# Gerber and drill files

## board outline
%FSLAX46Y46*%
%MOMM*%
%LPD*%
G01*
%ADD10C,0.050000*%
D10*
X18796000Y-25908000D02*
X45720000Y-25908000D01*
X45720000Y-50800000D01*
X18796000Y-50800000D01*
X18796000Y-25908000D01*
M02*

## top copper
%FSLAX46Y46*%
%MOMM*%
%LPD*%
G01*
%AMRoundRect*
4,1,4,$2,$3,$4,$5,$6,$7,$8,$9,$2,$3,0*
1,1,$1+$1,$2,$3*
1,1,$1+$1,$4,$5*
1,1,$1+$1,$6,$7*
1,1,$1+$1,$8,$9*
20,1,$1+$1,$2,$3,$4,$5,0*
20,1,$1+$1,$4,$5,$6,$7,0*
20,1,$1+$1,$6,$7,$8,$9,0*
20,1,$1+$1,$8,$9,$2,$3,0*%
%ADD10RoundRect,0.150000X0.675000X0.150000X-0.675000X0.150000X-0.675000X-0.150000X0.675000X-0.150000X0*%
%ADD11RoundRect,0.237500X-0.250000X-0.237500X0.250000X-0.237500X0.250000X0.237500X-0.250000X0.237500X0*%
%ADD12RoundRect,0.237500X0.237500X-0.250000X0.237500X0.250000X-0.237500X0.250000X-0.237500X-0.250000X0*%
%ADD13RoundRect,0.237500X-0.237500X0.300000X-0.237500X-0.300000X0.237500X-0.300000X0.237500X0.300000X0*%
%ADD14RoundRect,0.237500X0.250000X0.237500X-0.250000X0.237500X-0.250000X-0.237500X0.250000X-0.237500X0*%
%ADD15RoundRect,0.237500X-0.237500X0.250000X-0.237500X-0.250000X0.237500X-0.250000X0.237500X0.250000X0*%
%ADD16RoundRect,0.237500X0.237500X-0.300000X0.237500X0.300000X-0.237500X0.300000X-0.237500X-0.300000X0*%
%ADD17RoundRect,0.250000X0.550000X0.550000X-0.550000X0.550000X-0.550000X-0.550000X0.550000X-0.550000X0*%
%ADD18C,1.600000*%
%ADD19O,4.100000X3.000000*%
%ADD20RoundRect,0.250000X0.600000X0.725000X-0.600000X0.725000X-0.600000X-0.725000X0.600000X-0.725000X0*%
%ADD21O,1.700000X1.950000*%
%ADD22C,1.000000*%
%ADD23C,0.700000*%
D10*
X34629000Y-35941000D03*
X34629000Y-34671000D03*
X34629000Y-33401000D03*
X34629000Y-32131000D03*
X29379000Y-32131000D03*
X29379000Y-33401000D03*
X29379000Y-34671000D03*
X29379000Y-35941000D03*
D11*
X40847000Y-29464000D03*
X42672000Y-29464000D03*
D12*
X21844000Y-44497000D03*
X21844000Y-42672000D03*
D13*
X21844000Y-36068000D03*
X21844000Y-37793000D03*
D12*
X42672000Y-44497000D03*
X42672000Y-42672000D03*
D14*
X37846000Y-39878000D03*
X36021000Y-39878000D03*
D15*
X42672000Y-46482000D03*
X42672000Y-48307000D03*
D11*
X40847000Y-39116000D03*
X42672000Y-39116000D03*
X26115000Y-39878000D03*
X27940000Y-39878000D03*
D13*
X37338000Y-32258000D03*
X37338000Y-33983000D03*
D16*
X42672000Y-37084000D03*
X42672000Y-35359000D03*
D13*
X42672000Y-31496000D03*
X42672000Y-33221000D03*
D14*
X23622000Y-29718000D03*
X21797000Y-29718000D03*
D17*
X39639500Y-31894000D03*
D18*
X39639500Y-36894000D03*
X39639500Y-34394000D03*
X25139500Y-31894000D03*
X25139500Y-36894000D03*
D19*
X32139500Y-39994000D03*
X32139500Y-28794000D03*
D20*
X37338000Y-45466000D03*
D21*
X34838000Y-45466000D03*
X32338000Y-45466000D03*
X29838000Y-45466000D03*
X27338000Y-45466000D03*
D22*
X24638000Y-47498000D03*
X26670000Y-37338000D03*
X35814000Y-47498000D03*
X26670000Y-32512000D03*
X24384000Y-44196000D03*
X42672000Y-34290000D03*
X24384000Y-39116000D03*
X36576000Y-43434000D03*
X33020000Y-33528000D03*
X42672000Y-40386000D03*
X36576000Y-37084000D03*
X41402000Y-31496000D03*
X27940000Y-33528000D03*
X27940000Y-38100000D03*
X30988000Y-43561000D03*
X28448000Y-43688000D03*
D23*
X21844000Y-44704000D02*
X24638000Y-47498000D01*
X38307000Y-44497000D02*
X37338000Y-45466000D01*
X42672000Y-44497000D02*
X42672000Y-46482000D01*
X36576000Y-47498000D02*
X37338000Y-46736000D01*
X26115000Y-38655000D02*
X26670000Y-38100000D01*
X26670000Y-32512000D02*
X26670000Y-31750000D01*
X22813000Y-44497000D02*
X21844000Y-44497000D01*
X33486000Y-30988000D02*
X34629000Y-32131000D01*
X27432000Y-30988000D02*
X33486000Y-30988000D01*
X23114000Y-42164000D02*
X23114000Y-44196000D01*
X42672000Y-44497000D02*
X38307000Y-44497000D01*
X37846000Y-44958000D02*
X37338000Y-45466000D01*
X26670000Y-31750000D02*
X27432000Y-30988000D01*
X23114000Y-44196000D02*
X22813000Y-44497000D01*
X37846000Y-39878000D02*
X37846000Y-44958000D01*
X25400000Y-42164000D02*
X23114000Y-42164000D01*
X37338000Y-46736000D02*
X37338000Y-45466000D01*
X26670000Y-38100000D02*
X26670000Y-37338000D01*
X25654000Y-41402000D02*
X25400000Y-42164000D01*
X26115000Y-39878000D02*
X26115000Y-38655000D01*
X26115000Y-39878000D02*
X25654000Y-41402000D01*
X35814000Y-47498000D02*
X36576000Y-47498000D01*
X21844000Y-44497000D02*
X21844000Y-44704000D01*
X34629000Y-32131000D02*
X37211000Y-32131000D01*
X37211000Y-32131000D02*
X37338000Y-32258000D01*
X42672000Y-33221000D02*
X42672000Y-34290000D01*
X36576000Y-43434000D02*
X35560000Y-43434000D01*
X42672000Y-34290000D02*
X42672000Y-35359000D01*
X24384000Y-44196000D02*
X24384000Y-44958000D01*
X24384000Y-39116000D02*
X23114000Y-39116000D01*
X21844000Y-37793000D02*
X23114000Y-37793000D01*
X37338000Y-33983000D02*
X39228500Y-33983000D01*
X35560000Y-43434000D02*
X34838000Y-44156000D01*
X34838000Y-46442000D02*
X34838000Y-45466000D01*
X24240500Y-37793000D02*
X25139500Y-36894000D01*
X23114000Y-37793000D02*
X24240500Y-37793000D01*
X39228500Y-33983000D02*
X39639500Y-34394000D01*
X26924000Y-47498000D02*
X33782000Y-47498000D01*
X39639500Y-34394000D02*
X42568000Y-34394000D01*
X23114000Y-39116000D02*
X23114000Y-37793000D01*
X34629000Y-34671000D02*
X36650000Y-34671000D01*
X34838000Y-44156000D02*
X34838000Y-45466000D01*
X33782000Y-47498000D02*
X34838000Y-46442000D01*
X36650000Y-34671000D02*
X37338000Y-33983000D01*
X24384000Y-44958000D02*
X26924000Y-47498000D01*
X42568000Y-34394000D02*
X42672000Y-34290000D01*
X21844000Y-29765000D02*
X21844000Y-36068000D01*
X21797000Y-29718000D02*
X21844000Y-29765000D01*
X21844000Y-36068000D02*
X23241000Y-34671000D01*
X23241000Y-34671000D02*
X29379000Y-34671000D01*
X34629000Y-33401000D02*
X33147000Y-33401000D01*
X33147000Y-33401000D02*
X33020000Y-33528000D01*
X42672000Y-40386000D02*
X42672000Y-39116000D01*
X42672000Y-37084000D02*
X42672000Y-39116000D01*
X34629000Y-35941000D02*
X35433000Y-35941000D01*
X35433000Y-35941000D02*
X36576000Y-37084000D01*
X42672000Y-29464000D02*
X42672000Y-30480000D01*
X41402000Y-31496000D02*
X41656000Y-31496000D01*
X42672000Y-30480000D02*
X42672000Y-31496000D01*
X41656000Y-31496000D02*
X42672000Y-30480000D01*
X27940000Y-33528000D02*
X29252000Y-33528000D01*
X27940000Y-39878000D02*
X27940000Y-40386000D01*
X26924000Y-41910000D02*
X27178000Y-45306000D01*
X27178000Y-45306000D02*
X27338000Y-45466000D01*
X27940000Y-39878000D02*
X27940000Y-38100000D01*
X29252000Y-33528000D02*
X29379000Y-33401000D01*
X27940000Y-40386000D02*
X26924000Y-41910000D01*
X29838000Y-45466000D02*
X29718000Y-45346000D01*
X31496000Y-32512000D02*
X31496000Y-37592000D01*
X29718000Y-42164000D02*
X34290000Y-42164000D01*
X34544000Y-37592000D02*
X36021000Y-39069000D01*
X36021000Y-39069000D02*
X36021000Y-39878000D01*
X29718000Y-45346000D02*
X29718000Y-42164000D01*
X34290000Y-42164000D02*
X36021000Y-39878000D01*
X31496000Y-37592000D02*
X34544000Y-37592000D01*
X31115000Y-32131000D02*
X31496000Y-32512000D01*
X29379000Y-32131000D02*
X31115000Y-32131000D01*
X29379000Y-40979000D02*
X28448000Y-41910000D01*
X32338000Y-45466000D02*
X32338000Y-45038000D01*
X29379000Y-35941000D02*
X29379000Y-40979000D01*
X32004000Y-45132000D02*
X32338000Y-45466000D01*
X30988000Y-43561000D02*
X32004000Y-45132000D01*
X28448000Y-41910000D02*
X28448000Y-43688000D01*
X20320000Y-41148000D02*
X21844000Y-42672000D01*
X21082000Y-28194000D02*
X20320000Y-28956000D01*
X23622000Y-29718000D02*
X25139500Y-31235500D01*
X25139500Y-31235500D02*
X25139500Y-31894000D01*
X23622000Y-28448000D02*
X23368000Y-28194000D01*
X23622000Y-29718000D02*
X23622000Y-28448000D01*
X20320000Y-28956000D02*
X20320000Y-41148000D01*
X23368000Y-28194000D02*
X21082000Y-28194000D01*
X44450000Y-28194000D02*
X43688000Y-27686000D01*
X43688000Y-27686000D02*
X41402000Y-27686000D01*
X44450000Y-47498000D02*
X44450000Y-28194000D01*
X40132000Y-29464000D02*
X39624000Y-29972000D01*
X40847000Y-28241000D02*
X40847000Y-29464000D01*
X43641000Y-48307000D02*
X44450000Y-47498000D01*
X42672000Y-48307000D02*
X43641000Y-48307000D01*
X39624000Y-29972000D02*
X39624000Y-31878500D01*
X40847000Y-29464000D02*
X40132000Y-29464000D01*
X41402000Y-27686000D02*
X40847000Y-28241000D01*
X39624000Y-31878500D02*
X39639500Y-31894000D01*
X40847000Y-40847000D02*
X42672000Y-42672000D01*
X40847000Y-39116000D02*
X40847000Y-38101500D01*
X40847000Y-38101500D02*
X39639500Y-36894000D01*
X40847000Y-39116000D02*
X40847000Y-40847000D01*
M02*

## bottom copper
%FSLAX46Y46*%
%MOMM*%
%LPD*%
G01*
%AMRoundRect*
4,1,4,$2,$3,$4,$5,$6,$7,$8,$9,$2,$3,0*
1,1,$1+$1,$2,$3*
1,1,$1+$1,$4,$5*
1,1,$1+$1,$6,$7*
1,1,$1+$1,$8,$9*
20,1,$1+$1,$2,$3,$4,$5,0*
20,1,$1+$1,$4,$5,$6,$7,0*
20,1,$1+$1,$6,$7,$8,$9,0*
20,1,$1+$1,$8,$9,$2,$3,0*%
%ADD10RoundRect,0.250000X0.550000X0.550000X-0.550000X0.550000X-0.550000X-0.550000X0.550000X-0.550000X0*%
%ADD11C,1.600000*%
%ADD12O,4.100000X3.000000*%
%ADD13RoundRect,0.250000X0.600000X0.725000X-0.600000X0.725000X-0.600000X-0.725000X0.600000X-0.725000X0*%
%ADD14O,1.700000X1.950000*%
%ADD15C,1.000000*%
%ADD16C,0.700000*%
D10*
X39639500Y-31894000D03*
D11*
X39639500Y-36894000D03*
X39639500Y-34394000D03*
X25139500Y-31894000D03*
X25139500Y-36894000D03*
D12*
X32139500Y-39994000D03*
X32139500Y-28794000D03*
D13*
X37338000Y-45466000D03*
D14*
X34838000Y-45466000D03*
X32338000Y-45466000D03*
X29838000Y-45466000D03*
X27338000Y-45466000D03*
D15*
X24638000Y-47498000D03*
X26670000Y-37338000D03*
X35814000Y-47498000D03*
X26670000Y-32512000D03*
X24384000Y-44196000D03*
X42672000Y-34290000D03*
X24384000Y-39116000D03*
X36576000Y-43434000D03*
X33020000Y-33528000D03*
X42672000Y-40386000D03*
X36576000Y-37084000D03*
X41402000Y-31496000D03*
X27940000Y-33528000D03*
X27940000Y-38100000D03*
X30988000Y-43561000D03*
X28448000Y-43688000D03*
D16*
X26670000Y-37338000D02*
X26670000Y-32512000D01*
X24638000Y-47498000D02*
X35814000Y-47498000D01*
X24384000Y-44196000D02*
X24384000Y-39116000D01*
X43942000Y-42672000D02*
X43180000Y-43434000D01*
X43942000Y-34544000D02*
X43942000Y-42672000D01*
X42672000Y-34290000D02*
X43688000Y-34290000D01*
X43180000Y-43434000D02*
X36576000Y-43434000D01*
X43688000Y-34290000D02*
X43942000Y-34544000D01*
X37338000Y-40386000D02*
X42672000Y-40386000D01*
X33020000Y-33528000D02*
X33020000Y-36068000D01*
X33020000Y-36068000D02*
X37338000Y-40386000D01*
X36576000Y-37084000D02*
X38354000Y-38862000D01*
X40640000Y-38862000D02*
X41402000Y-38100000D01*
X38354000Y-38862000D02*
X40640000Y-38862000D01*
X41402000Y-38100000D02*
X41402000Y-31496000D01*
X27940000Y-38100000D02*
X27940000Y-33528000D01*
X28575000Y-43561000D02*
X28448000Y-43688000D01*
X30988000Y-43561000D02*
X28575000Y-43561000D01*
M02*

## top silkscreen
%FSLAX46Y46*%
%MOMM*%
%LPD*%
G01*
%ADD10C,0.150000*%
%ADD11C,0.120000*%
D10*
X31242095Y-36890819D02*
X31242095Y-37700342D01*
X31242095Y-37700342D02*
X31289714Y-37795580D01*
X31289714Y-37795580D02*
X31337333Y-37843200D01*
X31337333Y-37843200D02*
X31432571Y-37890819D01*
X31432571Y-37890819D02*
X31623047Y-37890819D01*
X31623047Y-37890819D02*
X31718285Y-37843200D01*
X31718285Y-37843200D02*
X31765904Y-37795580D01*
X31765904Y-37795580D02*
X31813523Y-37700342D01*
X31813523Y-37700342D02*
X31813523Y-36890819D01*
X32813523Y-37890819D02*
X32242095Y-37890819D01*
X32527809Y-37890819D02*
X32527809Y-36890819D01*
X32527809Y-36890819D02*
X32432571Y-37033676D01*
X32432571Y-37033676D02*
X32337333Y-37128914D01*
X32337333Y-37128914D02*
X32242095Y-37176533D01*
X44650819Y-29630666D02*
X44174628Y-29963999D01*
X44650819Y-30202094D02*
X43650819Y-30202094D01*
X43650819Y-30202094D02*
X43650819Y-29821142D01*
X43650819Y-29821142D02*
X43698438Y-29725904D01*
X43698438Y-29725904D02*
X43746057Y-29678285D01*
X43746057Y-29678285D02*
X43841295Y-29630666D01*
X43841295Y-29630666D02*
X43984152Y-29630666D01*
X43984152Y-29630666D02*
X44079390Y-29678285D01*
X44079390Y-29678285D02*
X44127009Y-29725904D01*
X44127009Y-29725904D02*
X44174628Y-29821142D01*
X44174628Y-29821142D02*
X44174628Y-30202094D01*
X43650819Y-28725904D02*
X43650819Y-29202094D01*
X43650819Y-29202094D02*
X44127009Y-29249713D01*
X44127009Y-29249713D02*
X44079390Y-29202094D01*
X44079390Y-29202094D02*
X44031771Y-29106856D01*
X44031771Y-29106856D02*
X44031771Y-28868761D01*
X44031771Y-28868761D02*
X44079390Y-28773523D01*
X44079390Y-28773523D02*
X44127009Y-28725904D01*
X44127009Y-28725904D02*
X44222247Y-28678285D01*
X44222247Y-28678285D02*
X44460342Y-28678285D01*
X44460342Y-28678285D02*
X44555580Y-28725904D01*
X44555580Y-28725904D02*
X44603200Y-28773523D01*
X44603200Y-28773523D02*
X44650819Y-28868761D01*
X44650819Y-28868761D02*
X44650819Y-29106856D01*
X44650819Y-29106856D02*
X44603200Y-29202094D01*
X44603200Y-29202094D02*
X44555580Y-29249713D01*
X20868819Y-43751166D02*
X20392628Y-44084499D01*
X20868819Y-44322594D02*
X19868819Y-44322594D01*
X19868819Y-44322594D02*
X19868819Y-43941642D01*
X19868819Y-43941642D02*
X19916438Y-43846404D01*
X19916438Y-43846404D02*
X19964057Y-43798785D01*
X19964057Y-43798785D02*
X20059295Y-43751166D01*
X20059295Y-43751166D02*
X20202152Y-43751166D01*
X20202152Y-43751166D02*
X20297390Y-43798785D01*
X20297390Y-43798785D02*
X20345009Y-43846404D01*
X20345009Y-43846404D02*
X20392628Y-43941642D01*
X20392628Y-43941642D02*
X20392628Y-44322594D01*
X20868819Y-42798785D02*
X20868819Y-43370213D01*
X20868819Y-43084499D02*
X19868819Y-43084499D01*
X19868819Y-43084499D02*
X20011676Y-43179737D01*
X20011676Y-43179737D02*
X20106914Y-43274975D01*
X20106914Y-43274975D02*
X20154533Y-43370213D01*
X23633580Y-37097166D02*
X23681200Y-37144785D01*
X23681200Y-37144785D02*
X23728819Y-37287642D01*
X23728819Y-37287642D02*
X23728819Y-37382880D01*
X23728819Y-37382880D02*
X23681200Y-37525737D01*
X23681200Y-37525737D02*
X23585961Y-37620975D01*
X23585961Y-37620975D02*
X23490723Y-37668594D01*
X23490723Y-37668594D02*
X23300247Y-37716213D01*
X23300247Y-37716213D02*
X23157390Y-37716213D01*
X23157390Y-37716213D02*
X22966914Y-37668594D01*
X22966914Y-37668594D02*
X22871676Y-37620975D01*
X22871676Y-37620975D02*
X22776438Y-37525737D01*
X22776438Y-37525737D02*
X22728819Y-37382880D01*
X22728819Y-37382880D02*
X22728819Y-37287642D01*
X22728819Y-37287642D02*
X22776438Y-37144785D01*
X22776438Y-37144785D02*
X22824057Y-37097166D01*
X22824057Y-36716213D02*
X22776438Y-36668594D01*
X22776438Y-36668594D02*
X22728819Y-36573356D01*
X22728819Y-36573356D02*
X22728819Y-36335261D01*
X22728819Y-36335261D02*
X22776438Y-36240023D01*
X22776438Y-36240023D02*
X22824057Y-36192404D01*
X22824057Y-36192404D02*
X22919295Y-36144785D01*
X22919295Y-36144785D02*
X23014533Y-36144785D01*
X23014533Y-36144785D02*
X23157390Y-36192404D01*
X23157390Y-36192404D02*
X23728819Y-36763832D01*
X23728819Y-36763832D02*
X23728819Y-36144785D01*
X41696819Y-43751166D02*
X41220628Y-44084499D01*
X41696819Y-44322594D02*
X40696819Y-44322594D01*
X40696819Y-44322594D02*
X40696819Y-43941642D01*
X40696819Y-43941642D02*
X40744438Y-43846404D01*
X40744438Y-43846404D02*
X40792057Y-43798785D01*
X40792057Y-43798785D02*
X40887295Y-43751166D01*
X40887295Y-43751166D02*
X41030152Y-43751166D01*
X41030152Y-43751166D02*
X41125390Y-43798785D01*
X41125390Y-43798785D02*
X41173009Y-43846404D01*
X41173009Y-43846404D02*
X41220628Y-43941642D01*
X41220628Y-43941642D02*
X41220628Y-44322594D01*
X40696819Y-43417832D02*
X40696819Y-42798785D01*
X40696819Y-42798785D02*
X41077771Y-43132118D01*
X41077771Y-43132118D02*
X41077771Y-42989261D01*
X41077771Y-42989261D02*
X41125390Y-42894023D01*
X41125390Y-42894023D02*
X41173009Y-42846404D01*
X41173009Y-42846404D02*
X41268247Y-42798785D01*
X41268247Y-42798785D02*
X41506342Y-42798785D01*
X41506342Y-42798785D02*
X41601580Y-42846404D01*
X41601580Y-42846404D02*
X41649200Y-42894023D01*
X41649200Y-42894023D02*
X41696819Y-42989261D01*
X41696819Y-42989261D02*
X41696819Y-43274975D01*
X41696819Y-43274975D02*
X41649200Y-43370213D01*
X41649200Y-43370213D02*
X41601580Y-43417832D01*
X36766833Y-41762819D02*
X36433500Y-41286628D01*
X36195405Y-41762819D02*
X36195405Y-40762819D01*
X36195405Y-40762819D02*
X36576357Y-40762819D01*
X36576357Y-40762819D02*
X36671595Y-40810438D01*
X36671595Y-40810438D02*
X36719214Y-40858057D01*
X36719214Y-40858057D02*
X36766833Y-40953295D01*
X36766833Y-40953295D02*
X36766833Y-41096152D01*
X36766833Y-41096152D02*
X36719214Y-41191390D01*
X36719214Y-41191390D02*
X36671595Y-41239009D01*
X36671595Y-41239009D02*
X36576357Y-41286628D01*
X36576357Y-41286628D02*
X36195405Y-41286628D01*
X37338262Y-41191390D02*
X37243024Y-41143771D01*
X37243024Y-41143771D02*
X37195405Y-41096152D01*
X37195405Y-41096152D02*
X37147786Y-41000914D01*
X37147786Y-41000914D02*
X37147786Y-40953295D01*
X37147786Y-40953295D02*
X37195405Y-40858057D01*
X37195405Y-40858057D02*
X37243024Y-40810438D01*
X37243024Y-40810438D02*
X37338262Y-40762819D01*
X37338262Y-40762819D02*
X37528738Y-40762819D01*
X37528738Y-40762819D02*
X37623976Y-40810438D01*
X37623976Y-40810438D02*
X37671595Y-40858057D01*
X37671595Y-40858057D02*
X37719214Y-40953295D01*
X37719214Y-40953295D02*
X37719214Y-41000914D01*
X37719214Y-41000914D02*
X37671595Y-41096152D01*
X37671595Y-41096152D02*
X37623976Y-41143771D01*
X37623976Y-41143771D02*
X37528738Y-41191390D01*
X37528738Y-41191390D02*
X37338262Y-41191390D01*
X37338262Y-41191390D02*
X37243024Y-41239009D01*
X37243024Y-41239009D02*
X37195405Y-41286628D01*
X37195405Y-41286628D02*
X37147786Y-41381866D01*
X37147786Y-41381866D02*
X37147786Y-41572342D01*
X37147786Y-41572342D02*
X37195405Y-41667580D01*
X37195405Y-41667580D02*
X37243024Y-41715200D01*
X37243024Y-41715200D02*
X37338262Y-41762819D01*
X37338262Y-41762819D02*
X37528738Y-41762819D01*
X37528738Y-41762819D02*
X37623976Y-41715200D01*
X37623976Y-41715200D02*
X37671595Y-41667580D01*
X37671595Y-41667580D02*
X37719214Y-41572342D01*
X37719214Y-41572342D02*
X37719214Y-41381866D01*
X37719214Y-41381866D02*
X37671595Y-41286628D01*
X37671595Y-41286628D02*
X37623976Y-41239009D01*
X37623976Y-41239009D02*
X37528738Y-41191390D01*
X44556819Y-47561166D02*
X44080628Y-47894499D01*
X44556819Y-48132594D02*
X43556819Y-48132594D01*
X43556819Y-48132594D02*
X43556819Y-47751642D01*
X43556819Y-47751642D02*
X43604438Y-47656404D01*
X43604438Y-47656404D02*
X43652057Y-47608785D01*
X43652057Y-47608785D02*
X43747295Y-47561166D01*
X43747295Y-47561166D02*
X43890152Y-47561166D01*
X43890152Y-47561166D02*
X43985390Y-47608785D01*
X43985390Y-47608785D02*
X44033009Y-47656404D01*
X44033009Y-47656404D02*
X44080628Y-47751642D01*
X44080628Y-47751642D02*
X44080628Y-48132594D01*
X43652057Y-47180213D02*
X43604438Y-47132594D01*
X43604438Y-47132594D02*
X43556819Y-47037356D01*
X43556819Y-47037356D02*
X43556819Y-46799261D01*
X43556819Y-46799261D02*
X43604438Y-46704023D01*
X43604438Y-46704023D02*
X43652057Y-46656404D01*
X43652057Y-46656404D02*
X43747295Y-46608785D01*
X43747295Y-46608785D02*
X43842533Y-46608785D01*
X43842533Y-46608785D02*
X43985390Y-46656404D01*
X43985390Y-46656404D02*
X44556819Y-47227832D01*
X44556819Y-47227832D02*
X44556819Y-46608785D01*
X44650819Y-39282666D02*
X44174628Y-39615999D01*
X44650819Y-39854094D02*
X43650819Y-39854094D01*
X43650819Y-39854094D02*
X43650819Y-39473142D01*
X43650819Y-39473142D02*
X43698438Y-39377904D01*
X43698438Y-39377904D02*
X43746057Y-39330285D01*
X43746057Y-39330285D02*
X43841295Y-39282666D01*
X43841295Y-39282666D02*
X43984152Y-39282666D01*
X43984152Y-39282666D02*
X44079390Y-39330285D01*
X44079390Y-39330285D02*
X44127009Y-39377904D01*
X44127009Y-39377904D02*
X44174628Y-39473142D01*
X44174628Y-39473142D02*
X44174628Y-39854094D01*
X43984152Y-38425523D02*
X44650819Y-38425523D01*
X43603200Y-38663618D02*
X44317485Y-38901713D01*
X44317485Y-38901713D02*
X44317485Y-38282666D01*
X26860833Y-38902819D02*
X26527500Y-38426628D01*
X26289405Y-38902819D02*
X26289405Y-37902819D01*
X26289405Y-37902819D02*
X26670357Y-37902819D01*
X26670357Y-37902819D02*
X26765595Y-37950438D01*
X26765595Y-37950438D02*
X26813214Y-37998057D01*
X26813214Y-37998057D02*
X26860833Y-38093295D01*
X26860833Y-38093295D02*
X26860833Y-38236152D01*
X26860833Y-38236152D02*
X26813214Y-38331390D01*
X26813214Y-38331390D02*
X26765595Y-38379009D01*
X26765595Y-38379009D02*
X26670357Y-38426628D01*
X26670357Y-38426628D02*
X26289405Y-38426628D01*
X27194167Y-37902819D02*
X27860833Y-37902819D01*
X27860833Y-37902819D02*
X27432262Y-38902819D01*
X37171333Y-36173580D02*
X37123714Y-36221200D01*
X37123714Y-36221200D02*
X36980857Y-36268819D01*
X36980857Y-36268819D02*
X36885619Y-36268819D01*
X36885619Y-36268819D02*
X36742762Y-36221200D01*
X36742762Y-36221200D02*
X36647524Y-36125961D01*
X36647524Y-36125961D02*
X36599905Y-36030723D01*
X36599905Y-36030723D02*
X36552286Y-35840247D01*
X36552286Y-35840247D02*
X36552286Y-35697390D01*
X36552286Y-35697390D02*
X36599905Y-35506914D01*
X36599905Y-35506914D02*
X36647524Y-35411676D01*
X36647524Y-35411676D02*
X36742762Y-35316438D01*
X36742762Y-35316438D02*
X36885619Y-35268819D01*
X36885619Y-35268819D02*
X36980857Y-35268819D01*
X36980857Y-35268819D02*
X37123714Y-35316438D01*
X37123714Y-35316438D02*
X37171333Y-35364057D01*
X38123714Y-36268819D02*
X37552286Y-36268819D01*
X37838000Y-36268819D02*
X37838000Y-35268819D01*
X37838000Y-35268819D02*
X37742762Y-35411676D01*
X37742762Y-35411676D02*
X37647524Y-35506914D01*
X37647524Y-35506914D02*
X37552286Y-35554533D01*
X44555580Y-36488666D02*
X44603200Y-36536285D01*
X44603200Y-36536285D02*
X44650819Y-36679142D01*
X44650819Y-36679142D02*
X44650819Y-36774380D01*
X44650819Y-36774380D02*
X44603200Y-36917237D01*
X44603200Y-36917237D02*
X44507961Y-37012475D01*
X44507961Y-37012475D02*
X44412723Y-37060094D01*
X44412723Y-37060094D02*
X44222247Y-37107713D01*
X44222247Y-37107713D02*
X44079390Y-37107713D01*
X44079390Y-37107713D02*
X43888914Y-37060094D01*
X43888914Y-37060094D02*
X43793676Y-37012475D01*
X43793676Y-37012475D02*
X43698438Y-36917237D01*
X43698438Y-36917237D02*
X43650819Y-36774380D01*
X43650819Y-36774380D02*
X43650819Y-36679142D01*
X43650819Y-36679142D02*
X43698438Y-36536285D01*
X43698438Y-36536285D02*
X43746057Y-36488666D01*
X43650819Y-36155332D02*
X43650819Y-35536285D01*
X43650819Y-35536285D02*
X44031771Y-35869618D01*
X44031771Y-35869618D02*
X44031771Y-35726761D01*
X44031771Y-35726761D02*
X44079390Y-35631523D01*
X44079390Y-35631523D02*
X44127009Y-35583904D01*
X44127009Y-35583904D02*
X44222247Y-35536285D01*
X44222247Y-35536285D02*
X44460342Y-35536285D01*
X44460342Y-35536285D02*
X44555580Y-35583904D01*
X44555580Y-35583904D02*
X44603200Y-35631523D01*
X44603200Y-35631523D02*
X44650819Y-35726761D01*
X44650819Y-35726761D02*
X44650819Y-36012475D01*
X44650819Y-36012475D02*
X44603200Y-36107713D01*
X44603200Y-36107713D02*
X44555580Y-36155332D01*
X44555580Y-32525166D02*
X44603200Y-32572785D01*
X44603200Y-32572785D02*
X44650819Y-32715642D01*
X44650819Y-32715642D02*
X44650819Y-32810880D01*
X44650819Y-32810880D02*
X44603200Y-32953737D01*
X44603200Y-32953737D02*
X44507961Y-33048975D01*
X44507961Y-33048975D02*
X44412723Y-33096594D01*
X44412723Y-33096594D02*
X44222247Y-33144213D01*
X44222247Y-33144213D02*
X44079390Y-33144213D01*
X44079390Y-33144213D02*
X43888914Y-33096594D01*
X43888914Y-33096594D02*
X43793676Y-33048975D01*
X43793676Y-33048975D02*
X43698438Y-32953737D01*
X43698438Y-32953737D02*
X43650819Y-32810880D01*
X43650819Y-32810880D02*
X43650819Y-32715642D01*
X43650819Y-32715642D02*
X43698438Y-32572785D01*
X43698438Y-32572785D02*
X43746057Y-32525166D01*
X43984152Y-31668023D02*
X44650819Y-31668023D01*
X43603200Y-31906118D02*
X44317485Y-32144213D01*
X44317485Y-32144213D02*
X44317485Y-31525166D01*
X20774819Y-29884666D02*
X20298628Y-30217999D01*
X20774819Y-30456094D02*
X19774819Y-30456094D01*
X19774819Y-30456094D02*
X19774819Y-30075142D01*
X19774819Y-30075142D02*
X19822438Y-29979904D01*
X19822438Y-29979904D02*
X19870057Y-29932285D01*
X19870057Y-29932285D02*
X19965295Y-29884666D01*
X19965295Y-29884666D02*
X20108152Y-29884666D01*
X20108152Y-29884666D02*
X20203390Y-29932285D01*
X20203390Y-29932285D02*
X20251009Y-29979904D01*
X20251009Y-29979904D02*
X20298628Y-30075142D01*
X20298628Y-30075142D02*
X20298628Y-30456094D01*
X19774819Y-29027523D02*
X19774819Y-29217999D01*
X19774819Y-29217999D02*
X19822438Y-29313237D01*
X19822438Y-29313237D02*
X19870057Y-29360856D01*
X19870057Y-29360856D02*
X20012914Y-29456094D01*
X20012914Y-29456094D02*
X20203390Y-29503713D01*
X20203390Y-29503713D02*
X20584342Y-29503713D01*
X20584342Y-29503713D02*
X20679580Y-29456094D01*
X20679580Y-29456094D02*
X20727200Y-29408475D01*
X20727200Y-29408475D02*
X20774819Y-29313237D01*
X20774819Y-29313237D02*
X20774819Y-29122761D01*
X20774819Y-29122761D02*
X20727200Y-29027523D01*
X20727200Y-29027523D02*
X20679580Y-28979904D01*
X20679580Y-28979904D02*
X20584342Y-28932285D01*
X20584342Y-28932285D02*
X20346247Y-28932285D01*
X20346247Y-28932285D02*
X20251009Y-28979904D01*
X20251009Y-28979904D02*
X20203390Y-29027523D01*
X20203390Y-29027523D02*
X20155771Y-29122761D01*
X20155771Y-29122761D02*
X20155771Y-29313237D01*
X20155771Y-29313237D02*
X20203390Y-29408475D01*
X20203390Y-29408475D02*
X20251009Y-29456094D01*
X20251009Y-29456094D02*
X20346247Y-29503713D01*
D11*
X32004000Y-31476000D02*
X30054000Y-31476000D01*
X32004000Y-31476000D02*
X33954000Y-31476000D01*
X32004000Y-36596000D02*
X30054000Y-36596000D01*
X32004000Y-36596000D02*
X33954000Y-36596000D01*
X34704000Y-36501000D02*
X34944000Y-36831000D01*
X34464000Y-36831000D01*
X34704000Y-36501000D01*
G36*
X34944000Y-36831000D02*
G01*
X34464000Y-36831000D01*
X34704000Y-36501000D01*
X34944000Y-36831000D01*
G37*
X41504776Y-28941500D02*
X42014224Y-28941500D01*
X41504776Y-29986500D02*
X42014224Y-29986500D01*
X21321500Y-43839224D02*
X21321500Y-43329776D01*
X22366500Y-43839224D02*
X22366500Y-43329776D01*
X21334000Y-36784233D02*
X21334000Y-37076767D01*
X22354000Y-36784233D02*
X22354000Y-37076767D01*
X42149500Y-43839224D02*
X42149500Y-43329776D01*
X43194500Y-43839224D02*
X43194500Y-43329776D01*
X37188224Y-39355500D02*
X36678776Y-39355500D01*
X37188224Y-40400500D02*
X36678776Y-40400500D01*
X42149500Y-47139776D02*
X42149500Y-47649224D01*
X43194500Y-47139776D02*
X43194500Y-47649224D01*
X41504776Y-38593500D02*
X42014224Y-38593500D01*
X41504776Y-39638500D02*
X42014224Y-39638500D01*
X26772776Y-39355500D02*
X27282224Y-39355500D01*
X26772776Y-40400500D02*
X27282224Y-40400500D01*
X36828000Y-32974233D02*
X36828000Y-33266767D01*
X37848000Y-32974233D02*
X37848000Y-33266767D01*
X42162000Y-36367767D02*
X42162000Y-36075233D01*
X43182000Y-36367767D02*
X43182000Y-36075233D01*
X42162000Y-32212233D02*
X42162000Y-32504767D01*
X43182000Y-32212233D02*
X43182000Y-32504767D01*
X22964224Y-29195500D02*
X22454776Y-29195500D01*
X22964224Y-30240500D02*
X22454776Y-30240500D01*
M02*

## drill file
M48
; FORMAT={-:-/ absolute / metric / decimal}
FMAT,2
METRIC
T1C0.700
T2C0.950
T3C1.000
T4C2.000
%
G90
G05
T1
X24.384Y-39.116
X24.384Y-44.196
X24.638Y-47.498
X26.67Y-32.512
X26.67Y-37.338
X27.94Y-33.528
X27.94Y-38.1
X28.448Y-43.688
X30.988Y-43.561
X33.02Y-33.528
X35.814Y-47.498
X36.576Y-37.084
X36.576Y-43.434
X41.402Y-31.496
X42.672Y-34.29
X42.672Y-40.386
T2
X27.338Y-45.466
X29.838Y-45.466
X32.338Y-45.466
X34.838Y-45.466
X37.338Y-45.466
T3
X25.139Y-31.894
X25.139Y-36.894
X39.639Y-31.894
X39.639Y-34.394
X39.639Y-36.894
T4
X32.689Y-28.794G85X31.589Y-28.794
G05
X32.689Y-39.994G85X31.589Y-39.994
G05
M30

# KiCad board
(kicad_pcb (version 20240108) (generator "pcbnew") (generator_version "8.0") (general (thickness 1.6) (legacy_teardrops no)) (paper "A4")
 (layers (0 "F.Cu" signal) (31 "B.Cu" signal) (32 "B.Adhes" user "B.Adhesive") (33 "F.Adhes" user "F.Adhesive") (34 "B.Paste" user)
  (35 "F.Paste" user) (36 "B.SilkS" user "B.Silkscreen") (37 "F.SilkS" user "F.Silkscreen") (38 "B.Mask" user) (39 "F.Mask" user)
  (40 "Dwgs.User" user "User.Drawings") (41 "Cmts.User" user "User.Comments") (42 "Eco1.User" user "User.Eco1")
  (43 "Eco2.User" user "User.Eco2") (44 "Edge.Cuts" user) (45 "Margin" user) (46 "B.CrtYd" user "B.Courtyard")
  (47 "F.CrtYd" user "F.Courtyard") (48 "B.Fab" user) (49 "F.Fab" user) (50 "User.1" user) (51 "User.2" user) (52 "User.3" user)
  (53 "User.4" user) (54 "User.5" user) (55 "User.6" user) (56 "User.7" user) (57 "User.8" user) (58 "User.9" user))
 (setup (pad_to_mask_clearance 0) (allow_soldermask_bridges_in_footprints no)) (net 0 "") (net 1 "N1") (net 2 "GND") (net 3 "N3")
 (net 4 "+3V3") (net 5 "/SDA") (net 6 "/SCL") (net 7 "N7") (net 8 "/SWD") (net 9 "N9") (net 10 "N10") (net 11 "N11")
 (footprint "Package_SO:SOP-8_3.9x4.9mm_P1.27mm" (layer "F.Cu") (at 32.004 34.036 180)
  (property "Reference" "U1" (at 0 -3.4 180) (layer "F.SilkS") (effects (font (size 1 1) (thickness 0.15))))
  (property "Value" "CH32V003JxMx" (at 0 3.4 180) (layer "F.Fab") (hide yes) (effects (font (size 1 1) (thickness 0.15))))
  (fp_line (start 0 2.56) (end 1.95 2.56) (stroke (width 0.12) (type solid)) (layer "F.SilkS"))
  (fp_line (start 0 2.56) (end -1.95 2.56) (stroke (width 0.12) (type solid)) (layer "F.SilkS"))
  (fp_line (start 0 -2.56) (end 1.95 -2.56) (stroke (width 0.12) (type solid)) (layer "F.SilkS"))
  (fp_line (start 0 -2.56) (end -1.95 -2.56) (stroke (width 0.12) (type solid)) (layer "F.SilkS"))
  (fp_poly
   (pts (xy -2.7 -2.465) (xy -2.94 -2.795) (xy -2.46 -2.795) (xy -2.7 -2.465)) (stroke (width 0.12) (type solid)) (fill solid)
   (layer "F.SilkS"))
  (pad "1" smd roundrect (at -2.625 -1.905 180) (size 1.65 0.6) (layers "F.Cu" "F.Paste" "F.Mask") (roundrect_rratio 0.25) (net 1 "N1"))
  (pad "2" smd roundrect (at -2.625 -0.635 180) (size 1.65 0.6) (layers "F.Cu" "F.Paste" "F.Mask") (roundrect_rratio 0.25) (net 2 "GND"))
  (pad "3" smd roundrect (at -2.625 0.635 180) (size 1.65 0.6) (layers "F.Cu" "F.Paste" "F.Mask") (roundrect_rratio 0.25) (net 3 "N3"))
  (pad "4" smd roundrect (at -2.625 1.905 180) (size 1.65 0.6) (layers "F.Cu" "F.Paste" "F.Mask") (roundrect_rratio 0.25) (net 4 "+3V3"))
  (pad "5" smd roundrect (at 2.625 1.905 180) (size 1.65 0.6) (layers "F.Cu" "F.Paste" "F.Mask") (roundrect_rratio 0.25) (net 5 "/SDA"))
  (pad "6" smd roundrect (at 2.625 0.635 180) (size 1.65 0.6) (layers "F.Cu" "F.Paste" "F.Mask") (roundrect_rratio 0.25) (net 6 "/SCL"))
  (pad "7" smd roundrect (at 2.625 -0.635 180) (size 1.65 0.6) (layers "F.Cu" "F.Paste" "F.Mask") (roundrect_rratio 0.25) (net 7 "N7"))
  (pad "8" smd roundrect (at 2.625 -1.905 180) (size 1.65 0.6) (layers "F.Cu" "F.Paste" "F.Mask") (roundrect_rratio 0.25) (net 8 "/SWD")))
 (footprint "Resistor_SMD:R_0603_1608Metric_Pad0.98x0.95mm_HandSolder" (layer "F.Cu") (at 41.7595 29.464)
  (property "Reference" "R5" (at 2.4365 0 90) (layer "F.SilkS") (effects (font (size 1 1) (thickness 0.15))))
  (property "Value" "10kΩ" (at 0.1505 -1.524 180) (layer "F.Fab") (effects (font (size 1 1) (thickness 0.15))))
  (fp_line (start -0.254724 -0.5225) (end 0.254724 -0.5225) (stroke (width 0.12) (type solid)) (layer "F.SilkS"))
  (fp_line (start -0.254724 0.5225) (end 0.254724 0.5225) (stroke (width 0.12) (type solid)) (layer "F.SilkS"))
  (pad "1" smd roundrect (at -0.9125 0) (size 0.975 0.95) (layers "F.Cu" "F.Paste" "F.Mask") (roundrect_rratio 0.25) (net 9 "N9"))
  (pad "2" smd roundrect (at 0.9125 0) (size 0.975 0.95) (layers "F.Cu" "F.Paste" "F.Mask") (roundrect_rratio 0.25) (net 1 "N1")))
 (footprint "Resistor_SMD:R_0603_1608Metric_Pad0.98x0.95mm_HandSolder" (layer "F.Cu") (at 21.844 43.5845 90)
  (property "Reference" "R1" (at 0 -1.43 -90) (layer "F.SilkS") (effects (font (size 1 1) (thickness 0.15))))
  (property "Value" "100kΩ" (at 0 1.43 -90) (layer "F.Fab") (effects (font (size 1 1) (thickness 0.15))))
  (fp_line (start -0.254724 -0.5225) (end 0.254724 -0.5225) (stroke (width 0.12) (type solid)) (layer "F.SilkS"))
  (fp_line (start -0.254724 0.5225) (end 0.254724 0.5225) (stroke (width 0.12) (type solid)) (layer "F.SilkS"))
  (pad "1" smd roundrect (at -0.9125 0 90) (size 0.975 0.95) (layers "F.Cu" "F.Paste" "F.Mask") (roundrect_rratio 0.25) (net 4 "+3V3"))
  (pad "2" smd roundrect (at 0.9125 0 90) (size 0.975 0.95) (layers "F.Cu" "F.Paste" "F.Mask") (roundrect_rratio 0.25) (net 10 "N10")))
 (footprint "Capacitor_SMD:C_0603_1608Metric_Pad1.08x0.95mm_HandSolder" (layer "F.Cu") (at 21.844 36.9305 -90)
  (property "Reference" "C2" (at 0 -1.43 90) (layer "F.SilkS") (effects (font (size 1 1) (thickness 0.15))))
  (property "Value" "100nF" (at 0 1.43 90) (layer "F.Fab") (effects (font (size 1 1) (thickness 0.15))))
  (fp_line (start -0.146267 0.51) (end 0.146267 0.51) (stroke (width 0.12) (type solid)) (layer "F.SilkS"))
  (fp_line (start -0.146267 -0.51) (end 0.146267 -0.51) (stroke (width 0.12) (type solid)) (layer "F.SilkS"))
  (pad "1" smd roundrect (at -0.8625 0 270) (size 1.075 0.95) (layers "F.Cu" "F.Paste" "F.Mask") (roundrect_rratio 0.25) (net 7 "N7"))
  (pad "2" smd roundrect (at 0.8625 0 270) (size 1.075 0.95) (layers "F.Cu" "F.Paste" "F.Mask") (roundrect_rratio 0.25) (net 2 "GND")))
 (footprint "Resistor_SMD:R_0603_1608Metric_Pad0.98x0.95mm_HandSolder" (layer "F.Cu") (at 42.672 43.5845 90)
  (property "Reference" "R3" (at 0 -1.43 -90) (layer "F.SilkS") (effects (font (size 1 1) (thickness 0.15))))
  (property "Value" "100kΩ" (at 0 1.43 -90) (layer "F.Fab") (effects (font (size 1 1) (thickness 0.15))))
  (fp_line (start -0.254724 -0.5225) (end 0.254724 -0.5225) (stroke (width 0.12) (type solid)) (layer "F.SilkS"))
  (fp_line (start -0.254724 0.5225) (end 0.254724 0.5225) (stroke (width 0.12) (type solid)) (layer "F.SilkS"))
  (pad "1" smd roundrect (at -0.9125 0 90) (size 0.975 0.95) (layers "F.Cu" "F.Paste" "F.Mask") (roundrect_rratio 0.25) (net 4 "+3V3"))
  (pad "2" smd roundrect (at 0.9125 0 90) (size 0.975 0.95) (layers "F.Cu" "F.Paste" "F.Mask") (roundrect_rratio 0.25) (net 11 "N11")))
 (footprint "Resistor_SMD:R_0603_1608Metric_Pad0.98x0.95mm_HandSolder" (layer "F.Cu") (at 36.9335 39.878 180)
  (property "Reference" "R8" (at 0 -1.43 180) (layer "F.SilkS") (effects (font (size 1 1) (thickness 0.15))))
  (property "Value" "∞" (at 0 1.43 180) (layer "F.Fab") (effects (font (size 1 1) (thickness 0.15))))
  (fp_line (start -0.254724 0.5225) (end 0.254724 0.5225) (stroke (width 0.12) (type solid)) (layer "F.SilkS"))
  (fp_line (start -0.254724 -0.5225) (end 0.254724 -0.5225) (stroke (width 0.12) (type solid)) (layer "F.SilkS"))
  (pad "1" smd roundrect (at -0.9125 0 180) (size 0.975 0.95) (layers "F.Cu" "F.Paste" "F.Mask") (roundrect_rratio 0.25) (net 4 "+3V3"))
  (pad "2" smd roundrect (at 0.9125 0 180) (size 0.975 0.95) (layers "F.Cu" "F.Paste" "F.Mask") (roundrect_rratio 0.25) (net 5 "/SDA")))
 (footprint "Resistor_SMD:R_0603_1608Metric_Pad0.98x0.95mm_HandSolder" (layer "F.Cu") (at 42.672 47.3945 -90)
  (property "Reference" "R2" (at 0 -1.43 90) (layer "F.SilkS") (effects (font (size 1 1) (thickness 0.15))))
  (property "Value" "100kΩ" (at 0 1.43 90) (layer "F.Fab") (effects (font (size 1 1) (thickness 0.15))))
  (fp_line (start -0.254724 0.5225) (end 0.254724 0.5225) (stroke (width 0.12) (type solid)) (layer "F.SilkS"))
  (fp_line (start -0.254724 -0.5225) (end 0.254724 -0.5225) (stroke (width 0.12) (type solid)) (layer "F.SilkS"))
  (pad "1" smd roundrect (at -0.9125 0 270) (size 0.975 0.95) (layers "F.Cu" "F.Paste" "F.Mask") (roundrect_rratio 0.25) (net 4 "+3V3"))
  (pad "2" smd roundrect (at 0.9125 0 270) (size 0.975 0.95) (layers "F.Cu" "F.Paste" "F.Mask") (roundrect_rratio 0.25) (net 9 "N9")))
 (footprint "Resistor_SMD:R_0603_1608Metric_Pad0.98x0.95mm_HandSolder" (layer "F.Cu") (at 41.7595 39.116)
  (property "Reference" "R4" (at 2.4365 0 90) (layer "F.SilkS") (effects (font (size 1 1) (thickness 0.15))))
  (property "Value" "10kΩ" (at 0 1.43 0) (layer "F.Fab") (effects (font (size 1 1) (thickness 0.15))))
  (fp_line (start -0.254724 -0.5225) (end 0.254724 -0.5225) (stroke (width 0.12) (type solid)) (layer "F.SilkS"))
  (fp_line (start -0.254724 0.5225) (end 0.254724 0.5225) (stroke (width 0.12) (type solid)) (layer "F.SilkS"))
  (pad "1" smd roundrect (at -0.9125 0) (size 0.975 0.95) (layers "F.Cu" "F.Paste" "F.Mask") (roundrect_rratio 0.25) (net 11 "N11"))
  (pad "2" smd roundrect (at 0.9125 0) (size 0.975 0.95) (layers "F.Cu" "F.Paste" "F.Mask") (roundrect_rratio 0.25) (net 3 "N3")))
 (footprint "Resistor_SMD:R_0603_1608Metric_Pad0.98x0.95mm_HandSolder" (layer "F.Cu") (at 27.0275 39.878)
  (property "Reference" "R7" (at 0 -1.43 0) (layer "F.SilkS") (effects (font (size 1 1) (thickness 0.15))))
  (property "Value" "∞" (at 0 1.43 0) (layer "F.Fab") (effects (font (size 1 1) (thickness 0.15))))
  (fp_line (start -0.254724 -0.5225) (end 0.254724 -0.5225) (stroke (width 0.12) (type solid)) (layer "F.SilkS"))
  (fp_line (start -0.254724 0.5225) (end 0.254724 0.5225) (stroke (width 0.12) (type solid)) (layer "F.SilkS"))
  (pad "1" smd roundrect (at -0.9125 0) (size 0.975 0.95) (layers "F.Cu" "F.Paste" "F.Mask") (roundrect_rratio 0.25) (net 4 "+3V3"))
  (pad "2" smd roundrect (at 0.9125 0) (size 0.975 0.95) (layers "F.Cu" "F.Paste" "F.Mask") (roundrect_rratio 0.25) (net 6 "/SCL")))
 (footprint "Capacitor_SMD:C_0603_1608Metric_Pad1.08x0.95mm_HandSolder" (layer "F.Cu") (at 37.338 33.1205 -90)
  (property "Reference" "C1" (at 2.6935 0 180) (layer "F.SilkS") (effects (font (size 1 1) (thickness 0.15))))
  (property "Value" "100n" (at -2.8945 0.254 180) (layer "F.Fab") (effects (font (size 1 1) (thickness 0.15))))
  (fp_line (start -0.146267 0.51) (end 0.146267 0.51) (stroke (width 0.12) (type solid)) (layer "F.SilkS"))
  (fp_line (start -0.146267 -0.51) (end 0.146267 -0.51) (stroke (width 0.12) (type solid)) (layer "F.SilkS"))
  (pad "1" smd roundrect (at -0.8625 0 270) (size 1.075 0.95) (layers "F.Cu" "F.Paste" "F.Mask") (roundrect_rratio 0.25) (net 4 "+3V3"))
  (pad "2" smd roundrect (at 0.8625 0 270) (size 1.075 0.95) (layers "F.Cu" "F.Paste" "F.Mask") (roundrect_rratio 0.25) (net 2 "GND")))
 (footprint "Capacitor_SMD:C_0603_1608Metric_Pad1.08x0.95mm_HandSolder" (layer "F.Cu") (at 42.672 36.2215 90)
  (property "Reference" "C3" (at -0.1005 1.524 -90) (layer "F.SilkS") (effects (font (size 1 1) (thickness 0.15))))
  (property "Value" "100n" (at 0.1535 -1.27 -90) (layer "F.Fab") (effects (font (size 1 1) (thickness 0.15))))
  (fp_line (start -0.146267 -0.51) (end 0.146267 -0.51) (stroke (width 0.12) (type solid)) (layer "F.SilkS"))
  (fp_line (start -0.146267 0.51) (end 0.146267 0.51) (stroke (width 0.12) (type solid)) (layer "F.SilkS"))
  (pad "1" smd roundrect (at -0.8625 0 90) (size 1.075 0.95) (layers "F.Cu" "F.Paste" "F.Mask") (roundrect_rratio 0.25) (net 3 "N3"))
  (pad "2" smd roundrect (at 0.8625 0 90) (size 1.075 0.95) (layers "F.Cu" "F.Paste" "F.Mask") (roundrect_rratio 0.25) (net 2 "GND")))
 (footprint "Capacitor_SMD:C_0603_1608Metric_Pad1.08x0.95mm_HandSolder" (layer "F.Cu") (at 42.672 32.3585 -90)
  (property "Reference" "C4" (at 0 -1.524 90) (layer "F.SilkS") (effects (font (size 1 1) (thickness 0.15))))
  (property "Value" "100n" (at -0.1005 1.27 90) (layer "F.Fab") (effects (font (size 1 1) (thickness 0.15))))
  (fp_line (start -0.146267 0.51) (end 0.146267 0.51) (stroke (width 0.12) (type solid)) (layer "F.SilkS"))
  (fp_line (start -0.146267 -0.51) (end 0.146267 -0.51) (stroke (width 0.12) (type solid)) (layer "F.SilkS"))
  (pad "1" smd roundrect (at -0.8625 0 270) (size 1.075 0.95) (layers "F.Cu" "F.Paste" "F.Mask") (roundrect_rratio 0.25) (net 1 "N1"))
  (pad "2" smd roundrect (at 0.8625 0 270) (size 1.075 0.95) (layers "F.Cu" "F.Paste" "F.Mask") (roundrect_rratio 0.25) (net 2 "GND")))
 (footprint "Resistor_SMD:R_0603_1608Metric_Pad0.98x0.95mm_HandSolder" (layer "F.Cu") (at 22.7095 29.718 180)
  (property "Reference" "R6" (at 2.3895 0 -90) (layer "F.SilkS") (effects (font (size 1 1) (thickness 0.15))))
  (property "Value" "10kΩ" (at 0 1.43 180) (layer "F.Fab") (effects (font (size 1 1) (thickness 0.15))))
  (fp_line (start -0.254724 0.5225) (end 0.254724 0.5225) (stroke (width 0.12) (type solid)) (layer "F.SilkS"))
  (fp_line (start -0.254724 -0.5225) (end 0.254724 -0.5225) (stroke (width 0.12) (type solid)) (layer "F.SilkS"))
  (pad "1" smd roundrect (at -0.9125 0 180) (size 0.975 0.95) (layers "F.Cu" "F.Paste" "F.Mask") (roundrect_rratio 0.25) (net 10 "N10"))
  (pad "2" smd roundrect (at 0.9125 0 180) (size 0.975 0.95) (layers "F.Cu" "F.Paste" "F.Mask") (roundrect_rratio 0.25) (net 7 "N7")))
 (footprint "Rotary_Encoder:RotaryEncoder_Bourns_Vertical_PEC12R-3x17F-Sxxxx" (layer "B.Cu") (at 39.6395 31.894 180)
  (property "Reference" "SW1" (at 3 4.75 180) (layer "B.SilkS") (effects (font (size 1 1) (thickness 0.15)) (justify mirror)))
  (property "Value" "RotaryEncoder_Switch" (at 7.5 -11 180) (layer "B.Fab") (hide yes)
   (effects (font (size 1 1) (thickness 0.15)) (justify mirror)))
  (pad "A" thru_hole roundrect (at 0 0 180) (size 1.6 1.6) (drill 1) (layers "*.Cu" "*.Mask") (remove_unused_layers no)
   (roundrect_rratio 0.15625) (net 9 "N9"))
  (pad "B" thru_hole circle (at 0 -5 180) (size 1.6 1.6) (drill 1) (layers "*.Cu" "*.Mask") (remove_unused_layers no) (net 11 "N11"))
  (pad "C" thru_hole circle (at 0 -2.5 180) (size 1.6 1.6) (drill 1) (layers "*.Cu" "*.Mask") (remove_unused_layers no) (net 2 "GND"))
  (pad "S1" thru_hole circle (at 14.5 0 180) (size 1.6 1.6) (drill 1) (layers "*.Cu" "*.Mask") (remove_unused_layers no) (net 10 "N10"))
  (pad "S2" thru_hole circle (at 14.5 -5 180) (size 1.6 1.6) (drill 1) (layers "*.Cu" "*.Mask") (remove_unused_layers no) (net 2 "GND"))
  (pad "SH" thru_hole oval (at 7.5 -8.1 180) (size 4.1 3) (drill oval 3.1 2) (layers "*.Cu" "*.Mask") (remove_unused_layers no))
  (pad "SH" thru_hole oval (at 7.5 3.1 180) (size 4.1 3) (drill oval 3.1 2) (layers "*.Cu" "*.Mask") (remove_unused_layers no)))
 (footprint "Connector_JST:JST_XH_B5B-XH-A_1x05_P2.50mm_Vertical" (layer "B.Cu") (at 37.338 45.466 180)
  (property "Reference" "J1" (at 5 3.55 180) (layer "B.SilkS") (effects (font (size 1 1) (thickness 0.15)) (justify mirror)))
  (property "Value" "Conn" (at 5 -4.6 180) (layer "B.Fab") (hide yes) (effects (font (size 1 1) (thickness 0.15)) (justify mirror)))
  (pad "1" thru_hole roundrect (at 0 0 180) (size 1.7 1.95) (drill 0.95) (layers "*.Cu" "*.Mask") (remove_unused_layers no)
   (roundrect_rratio 0.147059) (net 4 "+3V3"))
  (pad "2" thru_hole oval (at 2.5 0 180) (size 1.7 1.95) (drill 0.95) (layers "*.Cu" "*.Mask") (remove_unused_layers no) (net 2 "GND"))
  (pad "3" thru_hole oval (at 5 0 180) (size 1.7 1.95) (drill 0.95) (layers "*.Cu" "*.Mask") (remove_unused_layers no) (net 8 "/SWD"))
  (pad "4" thru_hole oval (at 7.5 0 180) (size 1.7 1.95) (drill 0.95) (layers "*.Cu" "*.Mask") (remove_unused_layers no) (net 5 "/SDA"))
  (pad "5" thru_hole oval (at 10 0 180) (size 1.7 1.95) (drill 0.95) (layers "*.Cu" "*.Mask") (remove_unused_layers no) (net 6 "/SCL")))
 (gr_rect (start 18.796 25.908) (end 45.72 50.8) (stroke (width 0.05) (type default)) (fill none) (layer "Edge.Cuts"))
 (segment (start 21.844 44.704) (end 24.638 47.498) (width 0.7) (layer "F.Cu") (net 4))
 (segment (start 38.307 44.497) (end 37.338 45.466) (width 0.7) (layer "F.Cu") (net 4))
 (segment (start 42.672 44.497) (end 42.672 46.482) (width 0.7) (layer "F.Cu") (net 4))
 (segment (start 36.576 47.498) (end 37.338 46.736) (width 0.7) (layer "F.Cu") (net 4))
 (segment (start 26.115 38.655) (end 26.67 38.1) (width 0.7) (layer "F.Cu") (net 4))
 (segment (start 26.67 32.512) (end 26.67 31.75) (width 0.7) (layer "F.Cu") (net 4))
 (segment (start 22.813 44.497) (end 21.844 44.497) (width 0.7) (layer "F.Cu") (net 4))
 (segment (start 33.486 30.988) (end 34.629 32.131) (width 0.7) (layer "F.Cu") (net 4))
 (segment (start 27.432 30.988) (end 33.486 30.988) (width 0.7) (layer "F.Cu") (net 4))
 (segment (start 23.114 42.164) (end 23.114 44.196) (width 0.7) (layer "F.Cu") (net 4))
 (segment (start 42.672 44.497) (end 38.307 44.497) (width 0.7) (layer "F.Cu") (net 4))
 (segment (start 37.846 44.958) (end 37.338 45.466) (width 0.7) (layer "F.Cu") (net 4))
 (segment (start 26.67 31.75) (end 27.432 30.988) (width 0.7) (layer "F.Cu") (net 4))
 (segment (start 23.114 44.196) (end 22.813 44.497) (width 0.7) (layer "F.Cu") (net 4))
 (segment (start 37.846 39.878) (end 37.846 44.958) (width 0.7) (layer "F.Cu") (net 4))
 (segment (start 25.4 42.164) (end 23.114 42.164) (width 0.7) (layer "F.Cu") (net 4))
 (segment (start 37.338 46.736) (end 37.338 45.466) (width 0.7) (layer "F.Cu") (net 4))
 (segment (start 26.67 38.1) (end 26.67 37.338) (width 0.7) (layer "F.Cu") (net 4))
 (segment (start 25.654 41.402) (end 25.4 42.164) (width 0.7) (layer "F.Cu") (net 4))
 (segment (start 26.115 39.878) (end 26.115 38.655) (width 0.7) (layer "F.Cu") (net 4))
 (segment (start 26.115 39.878) (end 25.654 41.402) (width 0.7) (layer "F.Cu") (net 4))
 (segment (start 35.814 47.498) (end 36.576 47.498) (width 0.7) (layer "F.Cu") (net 4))
 (segment (start 21.844 44.497) (end 21.844 44.704) (width 0.7) (layer "F.Cu") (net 4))
 (segment (start 34.629 32.131) (end 37.211 32.131) (width 0.7) (layer "F.Cu") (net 4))
 (segment (start 37.211 32.131) (end 37.338 32.258) (width 0.7) (layer "F.Cu") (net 4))
 (via (at 24.638 47.498) (size 1) (drill 0.7) (layers "F.Cu" "B.Cu") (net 4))
 (via (at 26.67 37.338) (size 1) (drill 0.7) (layers "F.Cu" "B.Cu") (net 4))
 (via (at 35.814 47.498) (size 1) (drill 0.7) (layers "F.Cu" "B.Cu") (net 4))
 (via (at 26.67 32.512) (size 1) (drill 0.7) (layers "F.Cu" "B.Cu") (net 4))
 (segment (start 26.67 37.338) (end 26.67 32.512) (width 0.7) (layer "B.Cu") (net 4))
 (segment (start 24.638 47.498) (end 35.814 47.498) (width 0.7) (layer "B.Cu") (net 4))
 (segment (start 42.672 33.221) (end 42.672 34.29) (width 0.7) (layer "F.Cu") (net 2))
 (segment (start 36.576 43.434) (end 35.56 43.434) (width 0.7) (layer "F.Cu") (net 2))
 (segment (start 42.672 34.29) (end 42.672 35.359) (width 0.7) (layer "F.Cu") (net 2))
 (segment (start 24.384 44.196) (end 24.384 44.958) (width 0.7) (layer "F.Cu") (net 2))
 (segment (start 24.384 39.116) (end 23.114 39.116) (width 0.7) (layer "F.Cu") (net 2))
 (segment (start 21.844 37.793) (end 23.114 37.793) (width 0.7) (layer "F.Cu") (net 2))
 (segment (start 37.338 33.983) (end 39.2285 33.983) (width 0.7) (layer "F.Cu") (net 2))
 (segment (start 35.56 43.434) (end 34.838 44.156) (width 0.7) (layer "F.Cu") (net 2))
 (segment (start 34.838 46.442) (end 34.838 45.466) (width 0.7) (layer "F.Cu") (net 2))
 (segment (start 24.2405 37.793) (end 25.1395 36.894) (width 0.7) (layer "F.Cu") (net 2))
 (segment (start 23.114 37.793) (end 24.2405 37.793) (width 0.7) (layer "F.Cu") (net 2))
 (segment (start 39.2285 33.983) (end 39.6395 34.394) (width 0.7) (layer "F.Cu") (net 2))
 (segment (start 26.924 47.498) (end 33.782 47.498) (width 0.7) (layer "F.Cu") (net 2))
 (segment (start 39.6395 34.394) (end 42.568 34.394) (width 0.7) (layer "F.Cu") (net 2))
 (segment (start 23.114 39.116) (end 23.114 37.793) (width 0.7) (layer "F.Cu") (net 2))
 (segment (start 34.629 34.671) (end 36.65 34.671) (width 0.7) (layer "F.Cu") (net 2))
 (segment (start 34.838 44.156) (end 34.838 45.466) (width 0.7) (layer "F.Cu") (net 2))
 (segment (start 33.782 47.498) (end 34.838 46.442) (width 0.7) (layer "F.Cu") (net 2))
 (segment (start 36.65 34.671) (end 37.338 33.983) (width 0.7) (layer "F.Cu") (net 2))
 (segment (start 24.384 44.958) (end 26.924 47.498) (width 0.7) (layer "F.Cu") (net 2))
 (segment (start 42.568 34.394) (end 42.672 34.29) (width 0.7) (layer "F.Cu") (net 2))
 (via (at 24.384 44.196) (size 1) (drill 0.7) (layers "F.Cu" "B.Cu") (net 2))
 (via (at 42.672 34.29) (size 1) (drill 0.7) (layers "F.Cu" "B.Cu") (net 2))
 (via (at 24.384 39.116) (size 1) (drill 0.7) (layers "F.Cu" "B.Cu") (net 2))
 (via (at 36.576 43.434) (size 1) (drill 0.7) (layers "F.Cu" "B.Cu") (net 2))
 (segment (start 24.384 44.196) (end 24.384 39.116) (width 0.7) (layer "B.Cu") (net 2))
 (segment (start 43.942 42.672) (end 43.18 43.434) (width 0.7) (layer "B.Cu") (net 2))
 (segment (start 43.942 34.544) (end 43.942 42.672) (width 0.7) (layer "B.Cu") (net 2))
 (segment (start 42.672 34.29) (end 43.688 34.29) (width 0.7) (layer "B.Cu") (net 2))
 (segment (start 43.18 43.434) (end 36.576 43.434) (width 0.7) (layer "B.Cu") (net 2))
 (segment (start 43.688 34.29) (end 43.942 34.544) (width 0.7) (layer "B.Cu") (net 2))
 (segment (start 21.844 29.765) (end 21.844 36.068) (width 0.7) (layer "F.Cu") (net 7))
 (segment (start 21.797 29.718) (end 21.844 29.765) (width 0.7) (layer "F.Cu") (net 7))
 (segment (start 21.844 36.068) (end 23.241 34.671) (width 0.7) (layer "F.Cu") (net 7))
 (segment (start 23.241 34.671) (end 29.379 34.671) (width 0.7) (layer "F.Cu") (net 7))
 (segment (start 34.629 33.401) (end 33.147 33.401) (width 0.7) (layer "F.Cu") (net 3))
 (segment (start 33.147 33.401) (end 33.02 33.528) (width 0.7) (layer "F.Cu") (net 3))
 (segment (start 42.672 40.386) (end 42.672 39.116) (width 0.7) (layer "F.Cu") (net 3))
 (segment (start 42.672 37.084) (end 42.672 39.116) (width 0.7) (layer "F.Cu") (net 3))
 (via (at 33.02 33.528) (size 1) (drill 0.7) (layers "F.Cu" "B.Cu") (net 3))
 (via (at 42.672 40.386) (size 1) (drill 0.7) (layers "F.Cu" "B.Cu") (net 3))
 (segment (start 37.338 40.386) (end 42.672 40.386) (width 0.7) (layer "B.Cu") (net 3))
 (segment (start 33.02 33.528) (end 33.02 36.068) (width 0.7) (layer "B.Cu") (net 3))
 (segment (start 33.02 36.068) (end 37.338 40.386) (width 0.7) (layer "B.Cu") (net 3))
 (segment (start 34.629 35.941) (end 35.433 35.941) (width 0.7) (layer "F.Cu") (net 1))
 (segment (start 35.433 35.941) (end 36.576 37.084) (width 0.7) (layer "F.Cu") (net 1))
 (segment (start 42.672 29.464) (end 42.672 30.48) (width 0.7) (layer "F.Cu") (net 1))
 (segment (start 41.402 31.496) (end 41.656 31.496) (width 0.7) (layer "F.Cu") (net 1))
 (segment (start 42.672 30.48) (end 42.672 31.496) (width 0.7) (layer "F.Cu") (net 1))
 (segment (start 41.656 31.496) (end 42.672 30.48) (width 0.7) (layer "F.Cu") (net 1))
 (via (at 36.576 37.084) (size 1) (drill 0.7) (layers "F.Cu" "B.Cu") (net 1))
 (via (at 41.402 31.496) (size 1) (drill 0.7) (layers "F.Cu" "B.Cu") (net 1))
 (segment (start 36.576 37.084) (end 38.354 38.862) (width 0.7) (layer "B.Cu") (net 1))
 (segment (start 40.64 38.862) (end 41.402 38.1) (width 0.7) (layer "B.Cu") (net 1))
 (segment (start 38.354 38.862) (end 40.64 38.862) (width 0.7) (layer "B.Cu") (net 1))
 (segment (start 41.402 38.1) (end 41.402 31.496) (width 0.7) (layer "B.Cu") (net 1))
 (segment (start 27.94 33.528) (end 29.252 33.528) (width 0.7) (layer "F.Cu") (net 6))
 (segment (start 27.94 39.878) (end 27.94 40.386) (width 0.7) (layer "F.Cu") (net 6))
 (segment (start 26.924 41.91) (end 27.178 45.306) (width 0.7) (layer "F.Cu") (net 6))
 (segment (start 27.178 45.306) (end 27.338 45.466) (width 0.7) (layer "F.Cu") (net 6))
 (segment (start 27.94 39.878) (end 27.94 38.1) (width 0.7) (layer "F.Cu") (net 6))
 (segment (start 29.252 33.528) (end 29.379 33.401) (width 0.7) (layer "F.Cu") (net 6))
 (segment (start 27.94 40.386) (end 26.924 41.91) (width 0.7) (layer "F.Cu") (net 6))
 (via (at 27.94 33.528) (size 1) (drill 0.7) (layers "F.Cu" "B.Cu") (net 6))
 (via (at 27.94 38.1) (size 1) (drill 0.7) (layers "F.Cu" "B.Cu") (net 6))
 (segment (start 27.94 38.1) (end 27.94 33.528) (width 0.7) (layer "B.Cu") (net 6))
 (segment (start 29.838 45.466) (end 29.718 45.346) (width 0.7) (layer "F.Cu") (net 5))
 (segment (start 31.496 32.512) (end 31.496 37.592) (width 0.7) (layer "F.Cu") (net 5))
 (segment (start 29.718 42.164) (end 34.29 42.164) (width 0.7) (layer "F.Cu") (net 5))
 (segment (start 34.544 37.592) (end 36.021 39.069) (width 0.7) (layer "F.Cu") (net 5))
 (segment (start 36.021 39.069) (end 36.021 39.878) (width 0.7) (layer "F.Cu") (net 5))
 (segment (start 29.718 45.346) (end 29.718 42.164) (width 0.7) (layer "F.Cu") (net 5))
 (segment (start 34.29 42.164) (end 36.021 39.878) (width 0.7) (layer "F.Cu") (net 5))
 (segment (start 31.496 37.592) (end 34.544 37.592) (width 0.7) (layer "F.Cu") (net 5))
 (segment (start 31.115 32.131) (end 31.496 32.512) (width 0.7) (layer "F.Cu") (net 5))
 (segment (start 29.379 32.131) (end 31.115 32.131) (width 0.7) (layer "F.Cu") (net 5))
 (segment (start 29.379 40.979) (end 28.448 41.91) (width 0.7) (layer "F.Cu") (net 8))
 (segment (start 32.338 45.466) (end 32.338 45.038) (width 0.7) (layer "F.Cu") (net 8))
 (segment (start 29.379 35.941) (end 29.379 40.979) (width 0.7) (layer "F.Cu") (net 8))
 (segment (start 32.004 45.132) (end 32.338 45.466) (width 0.7) (layer "F.Cu") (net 8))
 (segment (start 30.988 43.561) (end 32.004 45.132) (width 0.7) (layer "F.Cu") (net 8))
 (segment (start 28.448 41.91) (end 28.448 43.688) (width 0.7) (layer "F.Cu") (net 8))
 (via (at 30.988 43.561) (size 1) (drill 0.7) (layers "F.Cu" "B.Cu") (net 8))
 (via (at 28.448 43.688) (size 1) (drill 0.7) (layers "F.Cu" "B.Cu") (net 8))
 (segment (start 28.575 43.561) (end 28.448 43.688) (width 0.7) (layer "B.Cu") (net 8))
 (segment (start 30.988 43.561) (end 28.575 43.561) (width 0.7) (layer "B.Cu") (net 8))
 (segment (start 20.32 41.148) (end 21.844 42.672) (width 0.7) (layer "F.Cu") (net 10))
 (segment (start 21.082 28.194) (end 20.32 28.956) (width 0.7) (layer "F.Cu") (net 10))
 (segment (start 23.622 29.718) (end 25.1395 31.2355) (width 0.7) (layer "F.Cu") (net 10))
 (segment (start 25.1395 31.2355) (end 25.1395 31.894) (width 0.7) (layer "F.Cu") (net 10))
 (segment (start 23.622 28.448) (end 23.368 28.194) (width 0.7) (layer "F.Cu") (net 10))
 (segment (start 23.622 29.718) (end 23.622 28.448) (width 0.7) (layer "F.Cu") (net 10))
 (segment (start 20.32 28.956) (end 20.32 41.148) (width 0.7) (layer "F.Cu") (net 10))
 (segment (start 23.368 28.194) (end 21.082 28.194) (width 0.7) (layer "F.Cu") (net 10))
 (segment (start 44.45 28.194) (end 43.688 27.686) (width 0.7) (layer "F.Cu") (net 9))
 (segment (start 43.688 27.686) (end 41.402 27.686) (width 0.7) (layer "F.Cu") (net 9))
 (segment (start 44.45 47.498) (end 44.45 28.194) (width 0.7) (layer "F.Cu") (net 9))
 (segment (start 40.132 29.464) (end 39.624 29.972) (width 0.7) (layer "F.Cu") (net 9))
 (segment (start 40.847 28.241) (end 40.847 29.464) (width 0.7) (layer "F.Cu") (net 9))
 (segment (start 43.641 48.307) (end 44.45 47.498) (width 0.7) (layer "F.Cu") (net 9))
 (segment (start 42.672 48.307) (end 43.641 48.307) (width 0.7) (layer "F.Cu") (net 9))
 (segment (start 39.624 29.972) (end 39.624 31.8785) (width 0.7) (layer "F.Cu") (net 9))
 (segment (start 40.847 29.464) (end 40.132 29.464) (width 0.7) (layer "F.Cu") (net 9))
 (segment (start 41.402 27.686) (end 40.847 28.241) (width 0.7) (layer "F.Cu") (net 9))
 (segment (start 39.624 31.8785) (end 39.6395 31.894) (width 0.7) (layer "F.Cu") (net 9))
 (segment (start 40.847 40.847) (end 42.672 42.672) (width 0.7) (layer "F.Cu") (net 11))
 (segment (start 40.847 39.116) (end 40.847 38.1015) (width 0.7) (layer "F.Cu") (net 11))
 (segment (start 40.847 38.1015) (end 39.6395 36.894) (width 0.7) (layer "F.Cu") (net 11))
 (segment (start 40.847 39.116) (end 40.847 40.847) (width 0.7) (layer "F.Cu") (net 11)))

